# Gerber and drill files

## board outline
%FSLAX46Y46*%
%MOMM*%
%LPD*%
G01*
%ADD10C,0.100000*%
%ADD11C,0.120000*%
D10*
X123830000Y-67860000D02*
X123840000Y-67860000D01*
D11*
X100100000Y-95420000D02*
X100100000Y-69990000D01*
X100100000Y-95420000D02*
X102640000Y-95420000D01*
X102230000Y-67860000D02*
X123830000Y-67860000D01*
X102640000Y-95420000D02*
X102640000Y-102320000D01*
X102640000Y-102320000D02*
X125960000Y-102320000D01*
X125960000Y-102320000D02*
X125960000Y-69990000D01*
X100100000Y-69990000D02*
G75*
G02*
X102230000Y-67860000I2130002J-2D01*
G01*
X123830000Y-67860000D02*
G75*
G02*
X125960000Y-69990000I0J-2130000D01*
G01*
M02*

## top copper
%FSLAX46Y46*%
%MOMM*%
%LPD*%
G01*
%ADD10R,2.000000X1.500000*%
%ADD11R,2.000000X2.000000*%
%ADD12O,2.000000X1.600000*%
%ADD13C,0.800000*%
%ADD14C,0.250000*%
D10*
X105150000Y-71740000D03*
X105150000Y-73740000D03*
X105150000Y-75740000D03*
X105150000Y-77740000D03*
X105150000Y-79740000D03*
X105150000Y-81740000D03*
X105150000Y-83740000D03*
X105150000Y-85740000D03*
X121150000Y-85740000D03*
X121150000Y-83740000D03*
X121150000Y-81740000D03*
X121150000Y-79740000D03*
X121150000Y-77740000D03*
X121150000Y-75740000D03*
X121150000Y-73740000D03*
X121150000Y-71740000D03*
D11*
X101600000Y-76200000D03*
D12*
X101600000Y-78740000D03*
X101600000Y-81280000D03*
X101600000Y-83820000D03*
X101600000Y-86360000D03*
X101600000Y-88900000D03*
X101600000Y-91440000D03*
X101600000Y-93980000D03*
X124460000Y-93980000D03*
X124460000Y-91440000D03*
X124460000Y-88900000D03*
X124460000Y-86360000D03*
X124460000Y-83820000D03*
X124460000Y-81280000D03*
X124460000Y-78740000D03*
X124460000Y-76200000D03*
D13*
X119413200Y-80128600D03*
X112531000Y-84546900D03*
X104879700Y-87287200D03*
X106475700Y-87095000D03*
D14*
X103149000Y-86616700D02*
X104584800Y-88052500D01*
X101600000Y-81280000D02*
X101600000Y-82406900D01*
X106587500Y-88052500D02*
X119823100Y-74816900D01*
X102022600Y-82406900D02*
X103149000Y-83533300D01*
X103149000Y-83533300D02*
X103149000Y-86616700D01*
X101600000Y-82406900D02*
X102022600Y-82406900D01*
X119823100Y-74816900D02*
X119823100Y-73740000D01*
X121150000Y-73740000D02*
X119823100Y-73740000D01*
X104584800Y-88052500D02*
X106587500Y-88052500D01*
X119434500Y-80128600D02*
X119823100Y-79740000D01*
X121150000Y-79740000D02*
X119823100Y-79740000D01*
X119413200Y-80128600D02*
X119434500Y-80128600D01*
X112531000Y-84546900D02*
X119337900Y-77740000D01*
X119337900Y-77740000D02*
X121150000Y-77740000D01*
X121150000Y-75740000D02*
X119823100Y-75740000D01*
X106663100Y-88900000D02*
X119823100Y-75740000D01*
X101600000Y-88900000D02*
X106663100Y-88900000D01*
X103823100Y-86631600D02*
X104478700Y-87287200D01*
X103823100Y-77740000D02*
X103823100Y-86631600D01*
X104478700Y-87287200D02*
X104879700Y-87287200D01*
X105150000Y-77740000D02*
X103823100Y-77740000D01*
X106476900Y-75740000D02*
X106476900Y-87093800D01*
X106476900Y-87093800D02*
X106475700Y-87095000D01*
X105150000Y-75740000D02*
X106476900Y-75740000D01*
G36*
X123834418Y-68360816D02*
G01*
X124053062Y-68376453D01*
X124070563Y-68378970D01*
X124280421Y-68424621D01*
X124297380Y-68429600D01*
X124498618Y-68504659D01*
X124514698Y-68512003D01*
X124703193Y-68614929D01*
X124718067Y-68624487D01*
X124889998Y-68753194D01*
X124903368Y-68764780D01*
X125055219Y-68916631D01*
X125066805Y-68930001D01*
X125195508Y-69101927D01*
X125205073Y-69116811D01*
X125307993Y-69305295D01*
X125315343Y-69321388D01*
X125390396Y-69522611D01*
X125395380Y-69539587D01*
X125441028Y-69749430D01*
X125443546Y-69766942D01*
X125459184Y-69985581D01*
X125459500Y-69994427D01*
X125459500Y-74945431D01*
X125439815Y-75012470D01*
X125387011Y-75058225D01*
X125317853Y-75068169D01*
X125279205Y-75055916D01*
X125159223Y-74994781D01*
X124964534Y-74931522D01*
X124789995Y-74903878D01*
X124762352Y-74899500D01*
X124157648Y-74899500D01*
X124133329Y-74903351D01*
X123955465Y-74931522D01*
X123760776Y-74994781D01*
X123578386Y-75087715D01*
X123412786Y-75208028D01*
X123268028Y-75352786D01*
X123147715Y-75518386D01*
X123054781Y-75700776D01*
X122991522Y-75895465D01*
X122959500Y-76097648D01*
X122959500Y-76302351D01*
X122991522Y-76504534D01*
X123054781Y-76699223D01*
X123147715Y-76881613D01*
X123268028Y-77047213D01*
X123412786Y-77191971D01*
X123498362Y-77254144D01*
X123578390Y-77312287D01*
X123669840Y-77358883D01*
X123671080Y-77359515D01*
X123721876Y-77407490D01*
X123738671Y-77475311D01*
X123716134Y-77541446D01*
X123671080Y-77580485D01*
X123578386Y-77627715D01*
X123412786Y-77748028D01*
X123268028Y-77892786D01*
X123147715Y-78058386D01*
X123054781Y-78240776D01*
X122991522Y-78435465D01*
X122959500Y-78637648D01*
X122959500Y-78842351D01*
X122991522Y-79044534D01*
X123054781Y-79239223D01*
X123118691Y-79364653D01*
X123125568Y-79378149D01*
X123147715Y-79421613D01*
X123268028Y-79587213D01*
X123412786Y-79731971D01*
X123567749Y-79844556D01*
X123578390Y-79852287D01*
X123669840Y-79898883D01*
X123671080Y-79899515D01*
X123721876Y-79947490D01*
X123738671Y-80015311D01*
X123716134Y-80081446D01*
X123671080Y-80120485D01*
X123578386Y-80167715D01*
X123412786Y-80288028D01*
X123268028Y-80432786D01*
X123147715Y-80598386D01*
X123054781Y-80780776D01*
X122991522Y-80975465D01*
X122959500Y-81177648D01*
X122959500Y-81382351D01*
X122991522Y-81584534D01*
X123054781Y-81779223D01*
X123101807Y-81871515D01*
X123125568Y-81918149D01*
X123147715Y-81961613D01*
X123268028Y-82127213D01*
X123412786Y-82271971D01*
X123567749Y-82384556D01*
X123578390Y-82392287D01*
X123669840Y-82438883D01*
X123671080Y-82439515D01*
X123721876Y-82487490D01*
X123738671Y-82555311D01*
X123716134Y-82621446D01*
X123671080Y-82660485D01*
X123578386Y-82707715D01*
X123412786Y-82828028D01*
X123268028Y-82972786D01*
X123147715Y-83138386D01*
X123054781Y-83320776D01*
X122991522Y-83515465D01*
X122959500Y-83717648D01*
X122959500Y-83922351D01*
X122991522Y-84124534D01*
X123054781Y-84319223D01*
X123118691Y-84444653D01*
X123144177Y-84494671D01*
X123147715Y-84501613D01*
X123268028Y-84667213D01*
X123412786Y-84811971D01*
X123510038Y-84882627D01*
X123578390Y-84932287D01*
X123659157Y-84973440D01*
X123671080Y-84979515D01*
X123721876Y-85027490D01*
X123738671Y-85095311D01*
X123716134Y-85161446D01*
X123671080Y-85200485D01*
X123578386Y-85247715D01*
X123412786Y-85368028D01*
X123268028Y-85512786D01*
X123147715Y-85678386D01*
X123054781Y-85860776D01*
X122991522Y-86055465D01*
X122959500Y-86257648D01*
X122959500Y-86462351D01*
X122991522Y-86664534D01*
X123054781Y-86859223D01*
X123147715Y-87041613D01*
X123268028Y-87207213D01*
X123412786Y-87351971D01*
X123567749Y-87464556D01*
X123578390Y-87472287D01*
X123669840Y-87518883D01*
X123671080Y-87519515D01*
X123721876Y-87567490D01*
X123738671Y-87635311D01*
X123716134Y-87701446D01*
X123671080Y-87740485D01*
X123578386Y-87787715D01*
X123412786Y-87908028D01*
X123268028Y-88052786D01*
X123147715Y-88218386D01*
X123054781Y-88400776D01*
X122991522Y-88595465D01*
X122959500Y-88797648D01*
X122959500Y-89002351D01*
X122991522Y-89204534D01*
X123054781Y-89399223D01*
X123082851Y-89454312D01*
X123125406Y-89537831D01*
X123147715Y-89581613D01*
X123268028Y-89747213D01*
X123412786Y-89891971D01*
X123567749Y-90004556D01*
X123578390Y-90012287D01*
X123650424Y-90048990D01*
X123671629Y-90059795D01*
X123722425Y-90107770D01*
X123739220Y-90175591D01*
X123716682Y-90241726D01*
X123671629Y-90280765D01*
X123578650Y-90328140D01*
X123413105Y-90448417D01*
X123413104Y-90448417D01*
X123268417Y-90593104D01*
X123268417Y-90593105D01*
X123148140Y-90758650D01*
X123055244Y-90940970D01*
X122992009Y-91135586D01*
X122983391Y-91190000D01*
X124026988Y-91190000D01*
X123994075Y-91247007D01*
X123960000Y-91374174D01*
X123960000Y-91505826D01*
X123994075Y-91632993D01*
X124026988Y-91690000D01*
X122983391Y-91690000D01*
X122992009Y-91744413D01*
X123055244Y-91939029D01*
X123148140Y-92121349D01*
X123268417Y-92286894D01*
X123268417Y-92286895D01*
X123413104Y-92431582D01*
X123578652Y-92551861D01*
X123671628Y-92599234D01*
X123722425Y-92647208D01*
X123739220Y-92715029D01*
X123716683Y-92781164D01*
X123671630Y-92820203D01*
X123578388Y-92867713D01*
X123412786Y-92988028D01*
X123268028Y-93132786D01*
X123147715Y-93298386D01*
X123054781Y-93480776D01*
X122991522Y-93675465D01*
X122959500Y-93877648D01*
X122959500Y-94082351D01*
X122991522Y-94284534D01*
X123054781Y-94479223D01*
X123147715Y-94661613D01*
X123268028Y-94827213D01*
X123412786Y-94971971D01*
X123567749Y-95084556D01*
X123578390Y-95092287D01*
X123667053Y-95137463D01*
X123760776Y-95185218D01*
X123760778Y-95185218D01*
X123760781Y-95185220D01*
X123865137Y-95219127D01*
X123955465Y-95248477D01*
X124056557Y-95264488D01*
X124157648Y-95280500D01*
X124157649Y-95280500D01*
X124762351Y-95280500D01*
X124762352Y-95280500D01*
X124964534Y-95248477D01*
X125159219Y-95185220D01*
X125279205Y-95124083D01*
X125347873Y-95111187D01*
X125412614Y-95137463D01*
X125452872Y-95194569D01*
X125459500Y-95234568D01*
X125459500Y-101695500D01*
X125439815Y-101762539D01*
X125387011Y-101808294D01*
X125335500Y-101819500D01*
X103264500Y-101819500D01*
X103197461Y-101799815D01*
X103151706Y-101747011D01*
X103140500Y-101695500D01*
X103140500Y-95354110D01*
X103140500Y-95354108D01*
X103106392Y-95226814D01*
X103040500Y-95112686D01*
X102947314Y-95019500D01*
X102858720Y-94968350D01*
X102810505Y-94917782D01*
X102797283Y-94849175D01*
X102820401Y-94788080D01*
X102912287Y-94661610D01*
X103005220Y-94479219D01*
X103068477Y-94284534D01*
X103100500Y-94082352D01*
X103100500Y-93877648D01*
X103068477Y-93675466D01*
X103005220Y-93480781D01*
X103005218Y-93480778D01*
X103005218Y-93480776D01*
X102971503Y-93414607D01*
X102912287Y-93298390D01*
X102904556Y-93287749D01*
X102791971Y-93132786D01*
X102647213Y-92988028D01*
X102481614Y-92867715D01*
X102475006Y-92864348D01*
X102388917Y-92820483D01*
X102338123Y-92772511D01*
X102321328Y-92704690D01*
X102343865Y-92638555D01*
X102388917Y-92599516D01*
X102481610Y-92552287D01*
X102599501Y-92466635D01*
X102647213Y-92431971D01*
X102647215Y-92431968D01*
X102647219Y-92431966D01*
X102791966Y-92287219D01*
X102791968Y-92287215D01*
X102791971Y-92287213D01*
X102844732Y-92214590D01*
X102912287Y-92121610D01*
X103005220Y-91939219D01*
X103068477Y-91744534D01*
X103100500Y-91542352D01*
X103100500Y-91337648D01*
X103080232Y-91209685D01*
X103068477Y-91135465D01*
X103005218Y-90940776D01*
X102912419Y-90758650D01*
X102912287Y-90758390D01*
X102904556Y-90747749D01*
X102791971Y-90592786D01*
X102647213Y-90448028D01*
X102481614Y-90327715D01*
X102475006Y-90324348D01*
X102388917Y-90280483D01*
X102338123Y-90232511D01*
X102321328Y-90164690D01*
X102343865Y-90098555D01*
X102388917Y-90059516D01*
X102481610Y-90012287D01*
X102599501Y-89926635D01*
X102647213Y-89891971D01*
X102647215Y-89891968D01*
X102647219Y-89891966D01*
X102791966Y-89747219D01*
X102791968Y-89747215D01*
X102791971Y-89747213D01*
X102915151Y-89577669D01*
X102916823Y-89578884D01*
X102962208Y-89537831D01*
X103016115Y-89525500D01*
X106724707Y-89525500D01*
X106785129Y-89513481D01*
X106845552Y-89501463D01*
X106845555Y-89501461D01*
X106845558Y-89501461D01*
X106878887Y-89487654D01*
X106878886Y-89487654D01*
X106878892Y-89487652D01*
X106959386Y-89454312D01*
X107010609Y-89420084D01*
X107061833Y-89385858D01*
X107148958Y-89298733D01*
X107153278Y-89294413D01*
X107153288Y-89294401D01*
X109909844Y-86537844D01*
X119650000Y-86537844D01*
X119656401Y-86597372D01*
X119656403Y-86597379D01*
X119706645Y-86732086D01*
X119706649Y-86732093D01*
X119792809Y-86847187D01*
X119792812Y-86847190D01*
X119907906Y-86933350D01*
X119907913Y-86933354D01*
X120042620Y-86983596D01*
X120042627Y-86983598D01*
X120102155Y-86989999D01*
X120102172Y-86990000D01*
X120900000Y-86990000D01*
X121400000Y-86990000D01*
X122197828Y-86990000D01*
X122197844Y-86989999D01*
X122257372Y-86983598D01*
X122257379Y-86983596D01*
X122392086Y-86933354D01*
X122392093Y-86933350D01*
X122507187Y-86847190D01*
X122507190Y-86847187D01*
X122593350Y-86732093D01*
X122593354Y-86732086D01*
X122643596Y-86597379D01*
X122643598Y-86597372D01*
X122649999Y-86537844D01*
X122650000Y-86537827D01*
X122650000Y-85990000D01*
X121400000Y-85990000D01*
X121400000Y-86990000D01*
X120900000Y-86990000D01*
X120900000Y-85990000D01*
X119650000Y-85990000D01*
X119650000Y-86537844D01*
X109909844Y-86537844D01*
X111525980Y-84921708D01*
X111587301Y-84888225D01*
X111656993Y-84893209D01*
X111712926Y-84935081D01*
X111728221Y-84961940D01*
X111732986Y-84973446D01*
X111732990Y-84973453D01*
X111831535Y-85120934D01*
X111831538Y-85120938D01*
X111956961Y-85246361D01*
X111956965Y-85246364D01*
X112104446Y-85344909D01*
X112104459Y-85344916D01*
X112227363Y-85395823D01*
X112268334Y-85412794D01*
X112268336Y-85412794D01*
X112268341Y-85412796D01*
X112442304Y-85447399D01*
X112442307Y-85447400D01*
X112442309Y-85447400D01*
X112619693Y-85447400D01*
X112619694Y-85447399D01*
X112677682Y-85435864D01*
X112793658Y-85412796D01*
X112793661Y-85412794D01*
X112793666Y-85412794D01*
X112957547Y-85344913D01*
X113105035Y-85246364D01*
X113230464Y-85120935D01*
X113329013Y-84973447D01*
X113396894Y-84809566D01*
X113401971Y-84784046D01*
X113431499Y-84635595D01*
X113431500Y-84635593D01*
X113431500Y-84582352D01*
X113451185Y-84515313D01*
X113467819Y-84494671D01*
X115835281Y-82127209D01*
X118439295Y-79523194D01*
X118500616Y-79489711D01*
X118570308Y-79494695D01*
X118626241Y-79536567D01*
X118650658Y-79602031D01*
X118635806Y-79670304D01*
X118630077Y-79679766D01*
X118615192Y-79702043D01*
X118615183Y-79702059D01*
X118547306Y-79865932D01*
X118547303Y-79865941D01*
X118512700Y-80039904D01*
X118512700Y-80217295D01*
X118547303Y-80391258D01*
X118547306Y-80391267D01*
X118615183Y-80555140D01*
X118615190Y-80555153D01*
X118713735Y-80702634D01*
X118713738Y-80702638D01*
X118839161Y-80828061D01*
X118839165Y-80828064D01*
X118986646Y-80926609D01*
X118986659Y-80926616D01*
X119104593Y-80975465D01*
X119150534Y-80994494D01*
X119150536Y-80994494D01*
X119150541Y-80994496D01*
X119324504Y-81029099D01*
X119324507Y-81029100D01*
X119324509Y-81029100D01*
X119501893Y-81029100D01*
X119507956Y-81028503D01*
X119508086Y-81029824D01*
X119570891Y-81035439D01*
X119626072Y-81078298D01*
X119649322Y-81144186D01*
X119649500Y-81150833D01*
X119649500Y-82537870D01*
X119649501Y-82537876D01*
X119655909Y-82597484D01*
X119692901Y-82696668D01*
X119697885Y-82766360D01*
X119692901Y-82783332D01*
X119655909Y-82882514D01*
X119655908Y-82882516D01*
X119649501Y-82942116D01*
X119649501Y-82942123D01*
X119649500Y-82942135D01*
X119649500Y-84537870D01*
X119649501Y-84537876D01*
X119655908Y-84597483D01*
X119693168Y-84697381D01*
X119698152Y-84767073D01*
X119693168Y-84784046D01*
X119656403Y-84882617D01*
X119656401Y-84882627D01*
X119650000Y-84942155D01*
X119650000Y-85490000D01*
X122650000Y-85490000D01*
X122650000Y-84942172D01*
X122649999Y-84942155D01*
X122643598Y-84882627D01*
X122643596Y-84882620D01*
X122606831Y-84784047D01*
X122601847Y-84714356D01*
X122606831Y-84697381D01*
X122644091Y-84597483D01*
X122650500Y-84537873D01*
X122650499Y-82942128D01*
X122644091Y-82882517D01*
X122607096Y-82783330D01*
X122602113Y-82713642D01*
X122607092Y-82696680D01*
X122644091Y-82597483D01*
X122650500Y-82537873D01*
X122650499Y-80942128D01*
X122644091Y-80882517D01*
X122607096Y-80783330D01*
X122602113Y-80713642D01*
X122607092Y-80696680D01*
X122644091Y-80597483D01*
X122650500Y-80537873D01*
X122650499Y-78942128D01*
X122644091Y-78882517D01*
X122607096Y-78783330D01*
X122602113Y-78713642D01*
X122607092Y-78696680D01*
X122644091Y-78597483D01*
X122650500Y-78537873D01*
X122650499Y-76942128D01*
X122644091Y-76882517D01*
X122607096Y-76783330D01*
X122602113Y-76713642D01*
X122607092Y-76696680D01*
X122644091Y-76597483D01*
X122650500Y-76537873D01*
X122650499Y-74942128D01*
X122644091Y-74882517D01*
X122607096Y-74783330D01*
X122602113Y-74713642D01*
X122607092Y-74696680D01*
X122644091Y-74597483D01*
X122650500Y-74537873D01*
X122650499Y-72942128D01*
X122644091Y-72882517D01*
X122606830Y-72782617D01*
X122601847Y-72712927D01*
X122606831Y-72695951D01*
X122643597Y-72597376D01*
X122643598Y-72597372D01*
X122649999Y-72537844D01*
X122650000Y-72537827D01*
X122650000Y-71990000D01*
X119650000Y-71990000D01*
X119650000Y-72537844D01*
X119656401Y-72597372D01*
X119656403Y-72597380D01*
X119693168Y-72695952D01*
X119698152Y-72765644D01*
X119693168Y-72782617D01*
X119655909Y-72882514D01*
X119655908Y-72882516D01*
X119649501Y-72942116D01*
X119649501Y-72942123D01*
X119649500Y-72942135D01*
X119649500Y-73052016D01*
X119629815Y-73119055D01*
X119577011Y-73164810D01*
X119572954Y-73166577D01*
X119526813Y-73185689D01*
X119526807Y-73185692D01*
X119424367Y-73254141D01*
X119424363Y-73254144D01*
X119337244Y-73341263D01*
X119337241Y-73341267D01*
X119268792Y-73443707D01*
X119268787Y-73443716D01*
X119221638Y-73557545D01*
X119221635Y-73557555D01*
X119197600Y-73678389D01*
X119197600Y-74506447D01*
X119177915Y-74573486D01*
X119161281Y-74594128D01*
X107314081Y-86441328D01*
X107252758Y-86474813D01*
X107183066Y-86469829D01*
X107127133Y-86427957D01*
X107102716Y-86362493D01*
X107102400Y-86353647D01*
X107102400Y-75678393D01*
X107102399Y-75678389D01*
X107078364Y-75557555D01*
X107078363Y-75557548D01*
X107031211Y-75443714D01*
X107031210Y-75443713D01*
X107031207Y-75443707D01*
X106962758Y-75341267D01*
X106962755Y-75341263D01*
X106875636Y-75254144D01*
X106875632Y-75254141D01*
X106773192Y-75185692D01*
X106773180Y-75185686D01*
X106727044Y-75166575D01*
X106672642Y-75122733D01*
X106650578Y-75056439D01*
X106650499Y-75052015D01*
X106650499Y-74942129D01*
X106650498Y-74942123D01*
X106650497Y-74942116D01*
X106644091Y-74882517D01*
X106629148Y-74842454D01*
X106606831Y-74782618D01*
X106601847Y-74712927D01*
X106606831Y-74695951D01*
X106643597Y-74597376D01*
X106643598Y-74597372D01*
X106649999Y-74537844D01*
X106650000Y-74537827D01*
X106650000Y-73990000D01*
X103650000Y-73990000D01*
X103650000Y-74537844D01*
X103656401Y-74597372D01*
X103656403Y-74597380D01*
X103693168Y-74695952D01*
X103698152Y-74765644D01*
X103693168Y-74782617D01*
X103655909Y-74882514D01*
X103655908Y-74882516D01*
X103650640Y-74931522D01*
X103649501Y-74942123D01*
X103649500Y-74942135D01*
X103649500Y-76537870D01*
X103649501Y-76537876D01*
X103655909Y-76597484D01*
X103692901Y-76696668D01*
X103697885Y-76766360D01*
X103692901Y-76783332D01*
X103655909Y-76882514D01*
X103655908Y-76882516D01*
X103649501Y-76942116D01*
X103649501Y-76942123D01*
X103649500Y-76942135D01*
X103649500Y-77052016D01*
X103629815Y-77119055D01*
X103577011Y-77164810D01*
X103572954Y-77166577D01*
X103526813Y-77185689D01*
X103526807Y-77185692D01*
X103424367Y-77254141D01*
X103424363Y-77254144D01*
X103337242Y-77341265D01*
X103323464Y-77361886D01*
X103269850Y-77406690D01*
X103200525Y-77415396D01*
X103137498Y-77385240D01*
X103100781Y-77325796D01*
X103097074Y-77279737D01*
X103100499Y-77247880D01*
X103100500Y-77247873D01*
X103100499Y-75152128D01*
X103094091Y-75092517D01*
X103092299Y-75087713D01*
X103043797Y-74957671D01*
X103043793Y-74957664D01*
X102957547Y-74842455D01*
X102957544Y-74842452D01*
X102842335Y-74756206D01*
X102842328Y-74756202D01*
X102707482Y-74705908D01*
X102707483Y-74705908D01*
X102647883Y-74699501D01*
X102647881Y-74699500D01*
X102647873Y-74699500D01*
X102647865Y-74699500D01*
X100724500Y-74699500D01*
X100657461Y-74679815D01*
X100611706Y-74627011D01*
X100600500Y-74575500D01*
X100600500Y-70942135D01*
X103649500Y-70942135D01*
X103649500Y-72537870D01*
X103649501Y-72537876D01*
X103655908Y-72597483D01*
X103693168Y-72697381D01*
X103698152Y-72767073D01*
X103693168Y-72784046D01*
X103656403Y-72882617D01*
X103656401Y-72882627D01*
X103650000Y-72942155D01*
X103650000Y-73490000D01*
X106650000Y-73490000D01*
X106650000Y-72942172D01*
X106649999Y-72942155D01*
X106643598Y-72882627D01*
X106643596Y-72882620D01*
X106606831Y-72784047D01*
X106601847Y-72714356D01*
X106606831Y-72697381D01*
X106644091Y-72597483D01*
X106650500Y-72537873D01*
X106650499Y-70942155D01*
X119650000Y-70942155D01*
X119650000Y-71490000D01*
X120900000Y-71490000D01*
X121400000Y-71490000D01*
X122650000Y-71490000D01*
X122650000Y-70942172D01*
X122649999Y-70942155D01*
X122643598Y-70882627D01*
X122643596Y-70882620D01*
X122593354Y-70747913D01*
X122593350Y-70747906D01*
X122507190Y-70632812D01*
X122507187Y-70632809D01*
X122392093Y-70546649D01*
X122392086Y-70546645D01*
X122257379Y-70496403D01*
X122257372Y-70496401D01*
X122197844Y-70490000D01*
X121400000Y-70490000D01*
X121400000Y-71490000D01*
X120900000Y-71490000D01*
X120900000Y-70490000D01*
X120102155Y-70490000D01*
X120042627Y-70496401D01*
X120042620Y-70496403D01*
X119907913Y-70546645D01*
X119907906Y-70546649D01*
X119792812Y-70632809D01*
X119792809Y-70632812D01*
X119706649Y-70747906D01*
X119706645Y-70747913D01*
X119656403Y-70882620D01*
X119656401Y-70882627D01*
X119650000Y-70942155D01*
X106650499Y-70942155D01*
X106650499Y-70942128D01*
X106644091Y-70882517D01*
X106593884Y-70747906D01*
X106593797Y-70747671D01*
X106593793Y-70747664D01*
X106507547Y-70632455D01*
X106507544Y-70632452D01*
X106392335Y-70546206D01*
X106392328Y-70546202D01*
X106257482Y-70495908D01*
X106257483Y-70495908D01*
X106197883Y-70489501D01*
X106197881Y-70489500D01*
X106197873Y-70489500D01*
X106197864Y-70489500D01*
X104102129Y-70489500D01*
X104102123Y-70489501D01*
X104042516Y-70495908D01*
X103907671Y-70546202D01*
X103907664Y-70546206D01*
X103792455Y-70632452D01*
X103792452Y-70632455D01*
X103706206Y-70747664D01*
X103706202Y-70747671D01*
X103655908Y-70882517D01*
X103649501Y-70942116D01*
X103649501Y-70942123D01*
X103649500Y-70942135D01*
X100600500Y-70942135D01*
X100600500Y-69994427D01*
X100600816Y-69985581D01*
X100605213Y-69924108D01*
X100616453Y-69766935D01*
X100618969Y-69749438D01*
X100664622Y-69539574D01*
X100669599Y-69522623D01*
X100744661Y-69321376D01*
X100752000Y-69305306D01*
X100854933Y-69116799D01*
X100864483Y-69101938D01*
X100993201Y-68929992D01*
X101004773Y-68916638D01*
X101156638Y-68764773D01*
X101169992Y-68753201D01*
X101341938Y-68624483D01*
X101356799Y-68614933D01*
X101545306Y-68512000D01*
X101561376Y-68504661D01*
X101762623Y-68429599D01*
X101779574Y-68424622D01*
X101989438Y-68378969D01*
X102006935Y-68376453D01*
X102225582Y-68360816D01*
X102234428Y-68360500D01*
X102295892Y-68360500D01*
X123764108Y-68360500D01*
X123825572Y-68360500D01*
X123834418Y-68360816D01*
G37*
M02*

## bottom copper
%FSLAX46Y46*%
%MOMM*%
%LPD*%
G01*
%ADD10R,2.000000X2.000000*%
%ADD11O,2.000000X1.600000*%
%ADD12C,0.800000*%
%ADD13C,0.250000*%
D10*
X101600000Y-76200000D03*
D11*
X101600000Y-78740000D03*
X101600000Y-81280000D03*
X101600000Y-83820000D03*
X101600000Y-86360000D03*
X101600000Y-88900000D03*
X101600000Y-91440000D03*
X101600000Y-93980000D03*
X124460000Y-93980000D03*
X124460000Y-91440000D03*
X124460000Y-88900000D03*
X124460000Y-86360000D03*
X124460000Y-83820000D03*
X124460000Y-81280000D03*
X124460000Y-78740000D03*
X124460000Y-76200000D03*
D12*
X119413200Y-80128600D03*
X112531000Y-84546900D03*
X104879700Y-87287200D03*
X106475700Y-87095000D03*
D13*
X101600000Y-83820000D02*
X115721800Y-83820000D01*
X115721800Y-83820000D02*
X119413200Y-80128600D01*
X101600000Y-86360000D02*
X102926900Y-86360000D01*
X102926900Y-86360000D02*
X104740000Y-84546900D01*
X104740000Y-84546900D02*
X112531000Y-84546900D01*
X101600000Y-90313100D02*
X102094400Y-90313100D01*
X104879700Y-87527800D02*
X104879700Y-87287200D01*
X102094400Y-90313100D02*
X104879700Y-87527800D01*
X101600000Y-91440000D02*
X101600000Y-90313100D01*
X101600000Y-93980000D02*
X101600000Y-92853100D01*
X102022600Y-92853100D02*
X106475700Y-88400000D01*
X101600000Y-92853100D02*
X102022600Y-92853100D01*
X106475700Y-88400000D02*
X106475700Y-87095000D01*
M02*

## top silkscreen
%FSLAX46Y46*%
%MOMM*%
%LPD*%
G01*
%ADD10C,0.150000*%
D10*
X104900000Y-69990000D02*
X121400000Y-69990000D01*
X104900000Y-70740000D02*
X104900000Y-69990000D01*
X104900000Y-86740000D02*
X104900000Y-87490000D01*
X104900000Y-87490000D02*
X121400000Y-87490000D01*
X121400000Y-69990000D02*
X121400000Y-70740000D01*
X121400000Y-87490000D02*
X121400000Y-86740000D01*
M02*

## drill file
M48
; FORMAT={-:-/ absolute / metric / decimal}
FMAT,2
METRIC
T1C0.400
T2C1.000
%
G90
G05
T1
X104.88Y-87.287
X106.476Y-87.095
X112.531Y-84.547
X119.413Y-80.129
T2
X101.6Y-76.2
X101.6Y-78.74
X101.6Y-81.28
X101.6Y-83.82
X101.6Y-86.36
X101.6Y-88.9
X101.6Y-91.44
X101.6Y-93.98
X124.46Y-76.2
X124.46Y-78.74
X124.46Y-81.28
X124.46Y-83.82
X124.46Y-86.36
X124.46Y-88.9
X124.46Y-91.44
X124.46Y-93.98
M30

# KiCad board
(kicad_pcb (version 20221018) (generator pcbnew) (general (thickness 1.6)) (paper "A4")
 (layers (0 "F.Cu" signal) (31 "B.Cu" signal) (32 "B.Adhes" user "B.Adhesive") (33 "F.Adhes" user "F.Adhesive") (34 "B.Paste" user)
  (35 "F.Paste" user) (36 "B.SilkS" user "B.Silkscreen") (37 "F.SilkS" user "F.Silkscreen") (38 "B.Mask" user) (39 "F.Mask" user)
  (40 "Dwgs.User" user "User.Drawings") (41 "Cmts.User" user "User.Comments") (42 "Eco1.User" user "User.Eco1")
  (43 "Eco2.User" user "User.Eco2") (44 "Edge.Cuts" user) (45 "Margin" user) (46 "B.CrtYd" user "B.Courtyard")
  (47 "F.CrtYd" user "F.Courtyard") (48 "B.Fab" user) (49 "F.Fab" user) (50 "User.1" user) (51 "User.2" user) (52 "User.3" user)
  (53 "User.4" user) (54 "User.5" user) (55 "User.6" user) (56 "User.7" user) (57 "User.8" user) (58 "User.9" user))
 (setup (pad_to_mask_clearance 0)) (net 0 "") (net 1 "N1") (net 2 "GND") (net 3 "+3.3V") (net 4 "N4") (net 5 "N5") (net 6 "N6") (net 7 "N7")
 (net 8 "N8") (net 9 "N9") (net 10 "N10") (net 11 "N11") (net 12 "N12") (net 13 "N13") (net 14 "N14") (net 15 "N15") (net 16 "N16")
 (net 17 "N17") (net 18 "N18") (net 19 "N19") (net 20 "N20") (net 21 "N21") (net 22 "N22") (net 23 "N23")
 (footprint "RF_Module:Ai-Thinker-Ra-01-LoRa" (layer "F.Cu") (at 113.15 78.74)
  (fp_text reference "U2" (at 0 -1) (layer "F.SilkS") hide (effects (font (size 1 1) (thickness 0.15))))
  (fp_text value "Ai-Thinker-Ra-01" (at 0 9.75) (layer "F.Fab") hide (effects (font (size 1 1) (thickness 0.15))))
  (fp_line (start -8.25 -8.75) (end 8.25 -8.75) (stroke (width 0.15) (type solid)) (layer "F.SilkS"))
  (fp_line (start -8.25 -8) (end -8.25 -8.75) (stroke (width 0.15) (type solid)) (layer "F.SilkS"))
  (fp_line (start -8.25 8) (end -8.25 8.75) (stroke (width 0.15) (type solid)) (layer "F.SilkS"))
  (fp_line (start -8.25 8.75) (end 8.25 8.75) (stroke (width 0.15) (type solid)) (layer "F.SilkS"))
  (fp_line (start 8.25 -8.75) (end 8.25 -8) (stroke (width 0.15) (type solid)) (layer "F.SilkS"))
  (fp_line (start 8.25 8.75) (end 8.25 8) (stroke (width 0.15) (type solid)) (layer "F.SilkS"))
  (pad "1" smd rect (at -8 -7) (size 2 1.5) (layers "F.Cu" "F.Paste" "F.Mask") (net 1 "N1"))
  (pad "2" smd rect (at -8 -5) (size 2 1.5) (layers "F.Cu" "F.Paste" "F.Mask") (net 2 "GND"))
  (pad "3" smd rect (at -8 -3) (size 2 1.5) (layers "F.Cu" "F.Paste" "F.Mask") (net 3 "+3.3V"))
  (pad "4" smd rect (at -8 -1) (size 2 1.5) (layers "F.Cu" "F.Paste" "F.Mask") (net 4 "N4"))
  (pad "5" smd rect (at -8 1) (size 2 1.5) (layers "F.Cu" "F.Paste" "F.Mask") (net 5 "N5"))
  (pad "6" smd rect (at -8 3) (size 2 1.5) (layers "F.Cu" "F.Paste" "F.Mask") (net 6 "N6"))
  (pad "7" smd rect (at -8 5) (size 2 1.5) (layers "F.Cu" "F.Paste" "F.Mask") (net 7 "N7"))
  (pad "8" smd rect (at -8 7) (size 2 1.5) (layers "F.Cu" "F.Paste" "F.Mask") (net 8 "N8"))
  (pad "9" smd rect (at 8 7) (size 2 1.5) (layers "F.Cu" "F.Paste" "F.Mask") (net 2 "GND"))
  (pad "10" smd rect (at 8 5) (size 2 1.5) (layers "F.Cu" "F.Paste" "F.Mask") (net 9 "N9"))
  (pad "11" smd rect (at 8 3) (size 2 1.5) (layers "F.Cu" "F.Paste" "F.Mask") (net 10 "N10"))
  (pad "12" smd rect (at 8 1) (size 2 1.5) (layers "F.Cu" "F.Paste" "F.Mask") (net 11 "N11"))
  (pad "13" smd rect (at 8 -1) (size 2 1.5) (layers "F.Cu" "F.Paste" "F.Mask") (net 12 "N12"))
  (pad "14" smd rect (at 8 -3) (size 2 1.5) (layers "F.Cu" "F.Paste" "F.Mask") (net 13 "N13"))
  (pad "15" smd rect (at 8 -5) (size 2 1.5) (layers "F.Cu" "F.Paste" "F.Mask") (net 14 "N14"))
  (pad "16" smd rect (at 8 -7) (size 2 1.5) (layers "F.Cu" "F.Paste" "F.Mask") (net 2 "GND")))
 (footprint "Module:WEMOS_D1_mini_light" (layer "F.Cu") (at 101.6 76.2)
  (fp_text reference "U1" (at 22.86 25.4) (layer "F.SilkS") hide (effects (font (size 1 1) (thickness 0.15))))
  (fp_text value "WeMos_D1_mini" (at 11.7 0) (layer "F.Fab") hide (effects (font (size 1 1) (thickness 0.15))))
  (fp_line (start -1.5 19.22) (end -1.5 -6.21) (stroke (width 0.12) (type solid)) (layer "Edge.Cuts"))
  (fp_line (start -1.5 19.22) (end 1.04 19.22) (stroke (width 0.12) (type solid)) (layer "Edge.Cuts"))
  (fp_line (start 0.63 -8.34) (end 22.23 -8.34) (stroke (width 0.12) (type default)) (layer "Edge.Cuts"))
  (fp_line (start 1.04 19.22) (end 1.04 26.12) (stroke (width 0.12) (type solid)) (layer "Edge.Cuts"))
  (fp_line (start 1.04 26.12) (end 24.36 26.12) (stroke (width 0.12) (type solid)) (layer "Edge.Cuts"))
  (fp_line (start 24.36 26.12) (end 24.36 -6.21) (stroke (width 0.12) (type solid)) (layer "Edge.Cuts"))
  (fp_arc (start -1.5 -6.21) (mid -0.876137 -7.716137) (end 0.63 -8.34) (stroke (width 0.12) (type solid)) (layer "Edge.Cuts"))
  (fp_arc (start 22.23 -8.34) (mid 23.736137 -7.716137) (end 24.36 -6.21) (stroke (width 0.12) (type solid)) (layer "Edge.Cuts"))
  (pad "1" thru_hole rect (at 0 0) (size 2 2) (drill 1) (layers "*.Cu" "*.Mask") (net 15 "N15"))
  (pad "2" thru_hole oval (at 0 2.54) (size 2 1.6) (drill 1) (layers "*.Cu" "*.Mask") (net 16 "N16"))
  (pad "3" thru_hole oval (at 0 5.08) (size 2 1.6) (drill 1) (layers "*.Cu" "*.Mask") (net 14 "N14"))
  (pad "4" thru_hole oval (at 0 7.62) (size 2 1.6) (drill 1) (layers "*.Cu" "*.Mask") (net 11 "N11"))
  (pad "5" thru_hole oval (at 0 10.16) (size 2 1.6) (drill 1) (layers "*.Cu" "*.Mask") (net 12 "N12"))
  (pad "6" thru_hole oval (at 0 12.7) (size 2 1.6) (drill 1) (layers "*.Cu" "*.Mask") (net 13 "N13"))
  (pad "7" thru_hole oval (at 0 15.24) (size 2 1.6) (drill 1) (layers "*.Cu" "*.Mask") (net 4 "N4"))
  (pad "8" thru_hole oval (at 0 17.78) (size 2 1.6) (drill 1) (layers "*.Cu" "*.Mask") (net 3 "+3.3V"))
  (pad "9" thru_hole oval (at 22.86 17.78) (size 2 1.6) (drill 1) (layers "*.Cu" "*.Mask") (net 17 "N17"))
  (pad "10" thru_hole oval (at 22.86 15.24) (size 2 1.6) (drill 1) (layers "*.Cu" "*.Mask") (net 2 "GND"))
  (pad "11" thru_hole oval (at 22.86 12.7) (size 2 1.6) (drill 1) (layers "*.Cu" "*.Mask") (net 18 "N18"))
  (pad "12" thru_hole oval (at 22.86 10.16) (size 2 1.6) (drill 1) (layers "*.Cu" "*.Mask") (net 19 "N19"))
  (pad "13" thru_hole oval (at 22.86 7.62) (size 2 1.6) (drill 1) (layers "*.Cu" "*.Mask") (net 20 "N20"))
  (pad "14" thru_hole oval (at 22.86 5.08) (size 2 1.6) (drill 1) (layers "*.Cu" "*.Mask") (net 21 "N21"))
  (pad "15" thru_hole oval (at 22.86 2.54) (size 2 1.6) (drill 1) (layers "*.Cu" "*.Mask") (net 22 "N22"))
  (pad "16" thru_hole oval (at 22.86 0) (size 2 1.6) (drill 1) (layers "*.Cu" "*.Mask") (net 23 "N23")))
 (gr_line (start 123.83 67.86) (end 123.84 67.86) (stroke (width 0.1) (type default)) (layer "Edge.Cuts"))
 (segment (start 103.149 86.6167) (end 104.5848 88.0525) (width 0.25) (layer "F.Cu") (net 14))
 (segment (start 101.6 81.28) (end 101.6 82.4069) (width 0.25) (layer "F.Cu") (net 14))
 (segment (start 106.5875 88.0525) (end 119.8231 74.8169) (width 0.25) (layer "F.Cu") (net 14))
 (segment (start 102.0226 82.4069) (end 103.149 83.5333) (width 0.25) (layer "F.Cu") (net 14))
 (segment (start 103.149 83.5333) (end 103.149 86.6167) (width 0.25) (layer "F.Cu") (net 14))
 (segment (start 101.6 82.4069) (end 102.0226 82.4069) (width 0.25) (layer "F.Cu") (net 14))
 (segment (start 119.8231 74.8169) (end 119.8231 73.74) (width 0.25) (layer "F.Cu") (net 14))
 (segment (start 121.15 73.74) (end 119.8231 73.74) (width 0.25) (layer "F.Cu") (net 14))
 (segment (start 104.5848 88.0525) (end 106.5875 88.0525) (width 0.25) (layer "F.Cu") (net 14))
 (segment (start 119.4345 80.1286) (end 119.8231 79.74) (width 0.25) (layer "F.Cu") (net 11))
 (segment (start 121.15 79.74) (end 119.8231 79.74) (width 0.25) (layer "F.Cu") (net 11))
 (segment (start 119.4132 80.1286) (end 119.4345 80.1286) (width 0.25) (layer "F.Cu") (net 11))
 (via (at 119.4132 80.1286) (size 0.8) (drill 0.4) (layers "F.Cu" "B.Cu") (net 11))
 (segment (start 101.6 83.82) (end 115.7218 83.82) (width 0.25) (layer "B.Cu") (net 11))
 (segment (start 115.7218 83.82) (end 119.4132 80.1286) (width 0.25) (layer "B.Cu") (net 11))
 (segment (start 112.531 84.5469) (end 119.3379 77.74) (width 0.25) (layer "F.Cu") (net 12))
 (segment (start 119.3379 77.74) (end 121.15 77.74) (width 0.25) (layer "F.Cu") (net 12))
 (via (at 112.531 84.5469) (size 0.8) (drill 0.4) (layers "F.Cu" "B.Cu") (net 12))
 (segment (start 101.6 86.36) (end 102.9269 86.36) (width 0.25) (layer "B.Cu") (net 12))
 (segment (start 102.9269 86.36) (end 104.74 84.5469) (width 0.25) (layer "B.Cu") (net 12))
 (segment (start 104.74 84.5469) (end 112.531 84.5469) (width 0.25) (layer "B.Cu") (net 12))
 (segment (start 121.15 75.74) (end 119.8231 75.74) (width 0.25) (layer "F.Cu") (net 13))
 (segment (start 106.6631 88.9) (end 119.8231 75.74) (width 0.25) (layer "F.Cu") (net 13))
 (segment (start 101.6 88.9) (end 106.6631 88.9) (width 0.25) (layer "F.Cu") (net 13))
 (segment (start 103.8231 86.6316) (end 104.4787 87.2872) (width 0.25) (layer "F.Cu") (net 4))
 (segment (start 103.8231 77.74) (end 103.8231 86.6316) (width 0.25) (layer "F.Cu") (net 4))
 (segment (start 104.4787 87.2872) (end 104.8797 87.2872) (width 0.25) (layer "F.Cu") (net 4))
 (segment (start 105.15 77.74) (end 103.8231 77.74) (width 0.25) (layer "F.Cu") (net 4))
 (via (at 104.8797 87.2872) (size 0.8) (drill 0.4) (layers "F.Cu" "B.Cu") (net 4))
 (segment (start 101.6 90.3131) (end 102.0944 90.3131) (width 0.25) (layer "B.Cu") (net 4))
 (segment (start 104.8797 87.5278) (end 104.8797 87.2872) (width 0.25) (layer "B.Cu") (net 4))
 (segment (start 102.0944 90.3131) (end 104.8797 87.5278) (width 0.25) (layer "B.Cu") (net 4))
 (segment (start 101.6 91.44) (end 101.6 90.3131) (width 0.25) (layer "B.Cu") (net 4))
 (segment (start 106.4769 75.74) (end 106.4769 87.0938) (width 0.25) (layer "F.Cu") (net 3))
 (segment (start 106.4769 87.0938) (end 106.4757 87.095) (width 0.25) (layer "F.Cu") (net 3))
 (segment (start 105.15 75.74) (end 106.4769 75.74) (width 0.25) (layer "F.Cu") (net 3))
 (via (at 106.4757 87.095) (size 0.8) (drill 0.4) (layers "F.Cu" "B.Cu") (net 3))
 (segment (start 101.6 93.98) (end 101.6 92.8531) (width 0.25) (layer "B.Cu") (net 3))
 (segment (start 102.0226 92.8531) (end 106.4757 88.4) (width 0.25) (layer "B.Cu") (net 3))
 (segment (start 101.6 92.8531) (end 102.0226 92.8531) (width 0.25) (layer "B.Cu") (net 3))
 (segment (start 106.4757 88.4) (end 106.4757 87.095) (width 0.25) (layer "B.Cu") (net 3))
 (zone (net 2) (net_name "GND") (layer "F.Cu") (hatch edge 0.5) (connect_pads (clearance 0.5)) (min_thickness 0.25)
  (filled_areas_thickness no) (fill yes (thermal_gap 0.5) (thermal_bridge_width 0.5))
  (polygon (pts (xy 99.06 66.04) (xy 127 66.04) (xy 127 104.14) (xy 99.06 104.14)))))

